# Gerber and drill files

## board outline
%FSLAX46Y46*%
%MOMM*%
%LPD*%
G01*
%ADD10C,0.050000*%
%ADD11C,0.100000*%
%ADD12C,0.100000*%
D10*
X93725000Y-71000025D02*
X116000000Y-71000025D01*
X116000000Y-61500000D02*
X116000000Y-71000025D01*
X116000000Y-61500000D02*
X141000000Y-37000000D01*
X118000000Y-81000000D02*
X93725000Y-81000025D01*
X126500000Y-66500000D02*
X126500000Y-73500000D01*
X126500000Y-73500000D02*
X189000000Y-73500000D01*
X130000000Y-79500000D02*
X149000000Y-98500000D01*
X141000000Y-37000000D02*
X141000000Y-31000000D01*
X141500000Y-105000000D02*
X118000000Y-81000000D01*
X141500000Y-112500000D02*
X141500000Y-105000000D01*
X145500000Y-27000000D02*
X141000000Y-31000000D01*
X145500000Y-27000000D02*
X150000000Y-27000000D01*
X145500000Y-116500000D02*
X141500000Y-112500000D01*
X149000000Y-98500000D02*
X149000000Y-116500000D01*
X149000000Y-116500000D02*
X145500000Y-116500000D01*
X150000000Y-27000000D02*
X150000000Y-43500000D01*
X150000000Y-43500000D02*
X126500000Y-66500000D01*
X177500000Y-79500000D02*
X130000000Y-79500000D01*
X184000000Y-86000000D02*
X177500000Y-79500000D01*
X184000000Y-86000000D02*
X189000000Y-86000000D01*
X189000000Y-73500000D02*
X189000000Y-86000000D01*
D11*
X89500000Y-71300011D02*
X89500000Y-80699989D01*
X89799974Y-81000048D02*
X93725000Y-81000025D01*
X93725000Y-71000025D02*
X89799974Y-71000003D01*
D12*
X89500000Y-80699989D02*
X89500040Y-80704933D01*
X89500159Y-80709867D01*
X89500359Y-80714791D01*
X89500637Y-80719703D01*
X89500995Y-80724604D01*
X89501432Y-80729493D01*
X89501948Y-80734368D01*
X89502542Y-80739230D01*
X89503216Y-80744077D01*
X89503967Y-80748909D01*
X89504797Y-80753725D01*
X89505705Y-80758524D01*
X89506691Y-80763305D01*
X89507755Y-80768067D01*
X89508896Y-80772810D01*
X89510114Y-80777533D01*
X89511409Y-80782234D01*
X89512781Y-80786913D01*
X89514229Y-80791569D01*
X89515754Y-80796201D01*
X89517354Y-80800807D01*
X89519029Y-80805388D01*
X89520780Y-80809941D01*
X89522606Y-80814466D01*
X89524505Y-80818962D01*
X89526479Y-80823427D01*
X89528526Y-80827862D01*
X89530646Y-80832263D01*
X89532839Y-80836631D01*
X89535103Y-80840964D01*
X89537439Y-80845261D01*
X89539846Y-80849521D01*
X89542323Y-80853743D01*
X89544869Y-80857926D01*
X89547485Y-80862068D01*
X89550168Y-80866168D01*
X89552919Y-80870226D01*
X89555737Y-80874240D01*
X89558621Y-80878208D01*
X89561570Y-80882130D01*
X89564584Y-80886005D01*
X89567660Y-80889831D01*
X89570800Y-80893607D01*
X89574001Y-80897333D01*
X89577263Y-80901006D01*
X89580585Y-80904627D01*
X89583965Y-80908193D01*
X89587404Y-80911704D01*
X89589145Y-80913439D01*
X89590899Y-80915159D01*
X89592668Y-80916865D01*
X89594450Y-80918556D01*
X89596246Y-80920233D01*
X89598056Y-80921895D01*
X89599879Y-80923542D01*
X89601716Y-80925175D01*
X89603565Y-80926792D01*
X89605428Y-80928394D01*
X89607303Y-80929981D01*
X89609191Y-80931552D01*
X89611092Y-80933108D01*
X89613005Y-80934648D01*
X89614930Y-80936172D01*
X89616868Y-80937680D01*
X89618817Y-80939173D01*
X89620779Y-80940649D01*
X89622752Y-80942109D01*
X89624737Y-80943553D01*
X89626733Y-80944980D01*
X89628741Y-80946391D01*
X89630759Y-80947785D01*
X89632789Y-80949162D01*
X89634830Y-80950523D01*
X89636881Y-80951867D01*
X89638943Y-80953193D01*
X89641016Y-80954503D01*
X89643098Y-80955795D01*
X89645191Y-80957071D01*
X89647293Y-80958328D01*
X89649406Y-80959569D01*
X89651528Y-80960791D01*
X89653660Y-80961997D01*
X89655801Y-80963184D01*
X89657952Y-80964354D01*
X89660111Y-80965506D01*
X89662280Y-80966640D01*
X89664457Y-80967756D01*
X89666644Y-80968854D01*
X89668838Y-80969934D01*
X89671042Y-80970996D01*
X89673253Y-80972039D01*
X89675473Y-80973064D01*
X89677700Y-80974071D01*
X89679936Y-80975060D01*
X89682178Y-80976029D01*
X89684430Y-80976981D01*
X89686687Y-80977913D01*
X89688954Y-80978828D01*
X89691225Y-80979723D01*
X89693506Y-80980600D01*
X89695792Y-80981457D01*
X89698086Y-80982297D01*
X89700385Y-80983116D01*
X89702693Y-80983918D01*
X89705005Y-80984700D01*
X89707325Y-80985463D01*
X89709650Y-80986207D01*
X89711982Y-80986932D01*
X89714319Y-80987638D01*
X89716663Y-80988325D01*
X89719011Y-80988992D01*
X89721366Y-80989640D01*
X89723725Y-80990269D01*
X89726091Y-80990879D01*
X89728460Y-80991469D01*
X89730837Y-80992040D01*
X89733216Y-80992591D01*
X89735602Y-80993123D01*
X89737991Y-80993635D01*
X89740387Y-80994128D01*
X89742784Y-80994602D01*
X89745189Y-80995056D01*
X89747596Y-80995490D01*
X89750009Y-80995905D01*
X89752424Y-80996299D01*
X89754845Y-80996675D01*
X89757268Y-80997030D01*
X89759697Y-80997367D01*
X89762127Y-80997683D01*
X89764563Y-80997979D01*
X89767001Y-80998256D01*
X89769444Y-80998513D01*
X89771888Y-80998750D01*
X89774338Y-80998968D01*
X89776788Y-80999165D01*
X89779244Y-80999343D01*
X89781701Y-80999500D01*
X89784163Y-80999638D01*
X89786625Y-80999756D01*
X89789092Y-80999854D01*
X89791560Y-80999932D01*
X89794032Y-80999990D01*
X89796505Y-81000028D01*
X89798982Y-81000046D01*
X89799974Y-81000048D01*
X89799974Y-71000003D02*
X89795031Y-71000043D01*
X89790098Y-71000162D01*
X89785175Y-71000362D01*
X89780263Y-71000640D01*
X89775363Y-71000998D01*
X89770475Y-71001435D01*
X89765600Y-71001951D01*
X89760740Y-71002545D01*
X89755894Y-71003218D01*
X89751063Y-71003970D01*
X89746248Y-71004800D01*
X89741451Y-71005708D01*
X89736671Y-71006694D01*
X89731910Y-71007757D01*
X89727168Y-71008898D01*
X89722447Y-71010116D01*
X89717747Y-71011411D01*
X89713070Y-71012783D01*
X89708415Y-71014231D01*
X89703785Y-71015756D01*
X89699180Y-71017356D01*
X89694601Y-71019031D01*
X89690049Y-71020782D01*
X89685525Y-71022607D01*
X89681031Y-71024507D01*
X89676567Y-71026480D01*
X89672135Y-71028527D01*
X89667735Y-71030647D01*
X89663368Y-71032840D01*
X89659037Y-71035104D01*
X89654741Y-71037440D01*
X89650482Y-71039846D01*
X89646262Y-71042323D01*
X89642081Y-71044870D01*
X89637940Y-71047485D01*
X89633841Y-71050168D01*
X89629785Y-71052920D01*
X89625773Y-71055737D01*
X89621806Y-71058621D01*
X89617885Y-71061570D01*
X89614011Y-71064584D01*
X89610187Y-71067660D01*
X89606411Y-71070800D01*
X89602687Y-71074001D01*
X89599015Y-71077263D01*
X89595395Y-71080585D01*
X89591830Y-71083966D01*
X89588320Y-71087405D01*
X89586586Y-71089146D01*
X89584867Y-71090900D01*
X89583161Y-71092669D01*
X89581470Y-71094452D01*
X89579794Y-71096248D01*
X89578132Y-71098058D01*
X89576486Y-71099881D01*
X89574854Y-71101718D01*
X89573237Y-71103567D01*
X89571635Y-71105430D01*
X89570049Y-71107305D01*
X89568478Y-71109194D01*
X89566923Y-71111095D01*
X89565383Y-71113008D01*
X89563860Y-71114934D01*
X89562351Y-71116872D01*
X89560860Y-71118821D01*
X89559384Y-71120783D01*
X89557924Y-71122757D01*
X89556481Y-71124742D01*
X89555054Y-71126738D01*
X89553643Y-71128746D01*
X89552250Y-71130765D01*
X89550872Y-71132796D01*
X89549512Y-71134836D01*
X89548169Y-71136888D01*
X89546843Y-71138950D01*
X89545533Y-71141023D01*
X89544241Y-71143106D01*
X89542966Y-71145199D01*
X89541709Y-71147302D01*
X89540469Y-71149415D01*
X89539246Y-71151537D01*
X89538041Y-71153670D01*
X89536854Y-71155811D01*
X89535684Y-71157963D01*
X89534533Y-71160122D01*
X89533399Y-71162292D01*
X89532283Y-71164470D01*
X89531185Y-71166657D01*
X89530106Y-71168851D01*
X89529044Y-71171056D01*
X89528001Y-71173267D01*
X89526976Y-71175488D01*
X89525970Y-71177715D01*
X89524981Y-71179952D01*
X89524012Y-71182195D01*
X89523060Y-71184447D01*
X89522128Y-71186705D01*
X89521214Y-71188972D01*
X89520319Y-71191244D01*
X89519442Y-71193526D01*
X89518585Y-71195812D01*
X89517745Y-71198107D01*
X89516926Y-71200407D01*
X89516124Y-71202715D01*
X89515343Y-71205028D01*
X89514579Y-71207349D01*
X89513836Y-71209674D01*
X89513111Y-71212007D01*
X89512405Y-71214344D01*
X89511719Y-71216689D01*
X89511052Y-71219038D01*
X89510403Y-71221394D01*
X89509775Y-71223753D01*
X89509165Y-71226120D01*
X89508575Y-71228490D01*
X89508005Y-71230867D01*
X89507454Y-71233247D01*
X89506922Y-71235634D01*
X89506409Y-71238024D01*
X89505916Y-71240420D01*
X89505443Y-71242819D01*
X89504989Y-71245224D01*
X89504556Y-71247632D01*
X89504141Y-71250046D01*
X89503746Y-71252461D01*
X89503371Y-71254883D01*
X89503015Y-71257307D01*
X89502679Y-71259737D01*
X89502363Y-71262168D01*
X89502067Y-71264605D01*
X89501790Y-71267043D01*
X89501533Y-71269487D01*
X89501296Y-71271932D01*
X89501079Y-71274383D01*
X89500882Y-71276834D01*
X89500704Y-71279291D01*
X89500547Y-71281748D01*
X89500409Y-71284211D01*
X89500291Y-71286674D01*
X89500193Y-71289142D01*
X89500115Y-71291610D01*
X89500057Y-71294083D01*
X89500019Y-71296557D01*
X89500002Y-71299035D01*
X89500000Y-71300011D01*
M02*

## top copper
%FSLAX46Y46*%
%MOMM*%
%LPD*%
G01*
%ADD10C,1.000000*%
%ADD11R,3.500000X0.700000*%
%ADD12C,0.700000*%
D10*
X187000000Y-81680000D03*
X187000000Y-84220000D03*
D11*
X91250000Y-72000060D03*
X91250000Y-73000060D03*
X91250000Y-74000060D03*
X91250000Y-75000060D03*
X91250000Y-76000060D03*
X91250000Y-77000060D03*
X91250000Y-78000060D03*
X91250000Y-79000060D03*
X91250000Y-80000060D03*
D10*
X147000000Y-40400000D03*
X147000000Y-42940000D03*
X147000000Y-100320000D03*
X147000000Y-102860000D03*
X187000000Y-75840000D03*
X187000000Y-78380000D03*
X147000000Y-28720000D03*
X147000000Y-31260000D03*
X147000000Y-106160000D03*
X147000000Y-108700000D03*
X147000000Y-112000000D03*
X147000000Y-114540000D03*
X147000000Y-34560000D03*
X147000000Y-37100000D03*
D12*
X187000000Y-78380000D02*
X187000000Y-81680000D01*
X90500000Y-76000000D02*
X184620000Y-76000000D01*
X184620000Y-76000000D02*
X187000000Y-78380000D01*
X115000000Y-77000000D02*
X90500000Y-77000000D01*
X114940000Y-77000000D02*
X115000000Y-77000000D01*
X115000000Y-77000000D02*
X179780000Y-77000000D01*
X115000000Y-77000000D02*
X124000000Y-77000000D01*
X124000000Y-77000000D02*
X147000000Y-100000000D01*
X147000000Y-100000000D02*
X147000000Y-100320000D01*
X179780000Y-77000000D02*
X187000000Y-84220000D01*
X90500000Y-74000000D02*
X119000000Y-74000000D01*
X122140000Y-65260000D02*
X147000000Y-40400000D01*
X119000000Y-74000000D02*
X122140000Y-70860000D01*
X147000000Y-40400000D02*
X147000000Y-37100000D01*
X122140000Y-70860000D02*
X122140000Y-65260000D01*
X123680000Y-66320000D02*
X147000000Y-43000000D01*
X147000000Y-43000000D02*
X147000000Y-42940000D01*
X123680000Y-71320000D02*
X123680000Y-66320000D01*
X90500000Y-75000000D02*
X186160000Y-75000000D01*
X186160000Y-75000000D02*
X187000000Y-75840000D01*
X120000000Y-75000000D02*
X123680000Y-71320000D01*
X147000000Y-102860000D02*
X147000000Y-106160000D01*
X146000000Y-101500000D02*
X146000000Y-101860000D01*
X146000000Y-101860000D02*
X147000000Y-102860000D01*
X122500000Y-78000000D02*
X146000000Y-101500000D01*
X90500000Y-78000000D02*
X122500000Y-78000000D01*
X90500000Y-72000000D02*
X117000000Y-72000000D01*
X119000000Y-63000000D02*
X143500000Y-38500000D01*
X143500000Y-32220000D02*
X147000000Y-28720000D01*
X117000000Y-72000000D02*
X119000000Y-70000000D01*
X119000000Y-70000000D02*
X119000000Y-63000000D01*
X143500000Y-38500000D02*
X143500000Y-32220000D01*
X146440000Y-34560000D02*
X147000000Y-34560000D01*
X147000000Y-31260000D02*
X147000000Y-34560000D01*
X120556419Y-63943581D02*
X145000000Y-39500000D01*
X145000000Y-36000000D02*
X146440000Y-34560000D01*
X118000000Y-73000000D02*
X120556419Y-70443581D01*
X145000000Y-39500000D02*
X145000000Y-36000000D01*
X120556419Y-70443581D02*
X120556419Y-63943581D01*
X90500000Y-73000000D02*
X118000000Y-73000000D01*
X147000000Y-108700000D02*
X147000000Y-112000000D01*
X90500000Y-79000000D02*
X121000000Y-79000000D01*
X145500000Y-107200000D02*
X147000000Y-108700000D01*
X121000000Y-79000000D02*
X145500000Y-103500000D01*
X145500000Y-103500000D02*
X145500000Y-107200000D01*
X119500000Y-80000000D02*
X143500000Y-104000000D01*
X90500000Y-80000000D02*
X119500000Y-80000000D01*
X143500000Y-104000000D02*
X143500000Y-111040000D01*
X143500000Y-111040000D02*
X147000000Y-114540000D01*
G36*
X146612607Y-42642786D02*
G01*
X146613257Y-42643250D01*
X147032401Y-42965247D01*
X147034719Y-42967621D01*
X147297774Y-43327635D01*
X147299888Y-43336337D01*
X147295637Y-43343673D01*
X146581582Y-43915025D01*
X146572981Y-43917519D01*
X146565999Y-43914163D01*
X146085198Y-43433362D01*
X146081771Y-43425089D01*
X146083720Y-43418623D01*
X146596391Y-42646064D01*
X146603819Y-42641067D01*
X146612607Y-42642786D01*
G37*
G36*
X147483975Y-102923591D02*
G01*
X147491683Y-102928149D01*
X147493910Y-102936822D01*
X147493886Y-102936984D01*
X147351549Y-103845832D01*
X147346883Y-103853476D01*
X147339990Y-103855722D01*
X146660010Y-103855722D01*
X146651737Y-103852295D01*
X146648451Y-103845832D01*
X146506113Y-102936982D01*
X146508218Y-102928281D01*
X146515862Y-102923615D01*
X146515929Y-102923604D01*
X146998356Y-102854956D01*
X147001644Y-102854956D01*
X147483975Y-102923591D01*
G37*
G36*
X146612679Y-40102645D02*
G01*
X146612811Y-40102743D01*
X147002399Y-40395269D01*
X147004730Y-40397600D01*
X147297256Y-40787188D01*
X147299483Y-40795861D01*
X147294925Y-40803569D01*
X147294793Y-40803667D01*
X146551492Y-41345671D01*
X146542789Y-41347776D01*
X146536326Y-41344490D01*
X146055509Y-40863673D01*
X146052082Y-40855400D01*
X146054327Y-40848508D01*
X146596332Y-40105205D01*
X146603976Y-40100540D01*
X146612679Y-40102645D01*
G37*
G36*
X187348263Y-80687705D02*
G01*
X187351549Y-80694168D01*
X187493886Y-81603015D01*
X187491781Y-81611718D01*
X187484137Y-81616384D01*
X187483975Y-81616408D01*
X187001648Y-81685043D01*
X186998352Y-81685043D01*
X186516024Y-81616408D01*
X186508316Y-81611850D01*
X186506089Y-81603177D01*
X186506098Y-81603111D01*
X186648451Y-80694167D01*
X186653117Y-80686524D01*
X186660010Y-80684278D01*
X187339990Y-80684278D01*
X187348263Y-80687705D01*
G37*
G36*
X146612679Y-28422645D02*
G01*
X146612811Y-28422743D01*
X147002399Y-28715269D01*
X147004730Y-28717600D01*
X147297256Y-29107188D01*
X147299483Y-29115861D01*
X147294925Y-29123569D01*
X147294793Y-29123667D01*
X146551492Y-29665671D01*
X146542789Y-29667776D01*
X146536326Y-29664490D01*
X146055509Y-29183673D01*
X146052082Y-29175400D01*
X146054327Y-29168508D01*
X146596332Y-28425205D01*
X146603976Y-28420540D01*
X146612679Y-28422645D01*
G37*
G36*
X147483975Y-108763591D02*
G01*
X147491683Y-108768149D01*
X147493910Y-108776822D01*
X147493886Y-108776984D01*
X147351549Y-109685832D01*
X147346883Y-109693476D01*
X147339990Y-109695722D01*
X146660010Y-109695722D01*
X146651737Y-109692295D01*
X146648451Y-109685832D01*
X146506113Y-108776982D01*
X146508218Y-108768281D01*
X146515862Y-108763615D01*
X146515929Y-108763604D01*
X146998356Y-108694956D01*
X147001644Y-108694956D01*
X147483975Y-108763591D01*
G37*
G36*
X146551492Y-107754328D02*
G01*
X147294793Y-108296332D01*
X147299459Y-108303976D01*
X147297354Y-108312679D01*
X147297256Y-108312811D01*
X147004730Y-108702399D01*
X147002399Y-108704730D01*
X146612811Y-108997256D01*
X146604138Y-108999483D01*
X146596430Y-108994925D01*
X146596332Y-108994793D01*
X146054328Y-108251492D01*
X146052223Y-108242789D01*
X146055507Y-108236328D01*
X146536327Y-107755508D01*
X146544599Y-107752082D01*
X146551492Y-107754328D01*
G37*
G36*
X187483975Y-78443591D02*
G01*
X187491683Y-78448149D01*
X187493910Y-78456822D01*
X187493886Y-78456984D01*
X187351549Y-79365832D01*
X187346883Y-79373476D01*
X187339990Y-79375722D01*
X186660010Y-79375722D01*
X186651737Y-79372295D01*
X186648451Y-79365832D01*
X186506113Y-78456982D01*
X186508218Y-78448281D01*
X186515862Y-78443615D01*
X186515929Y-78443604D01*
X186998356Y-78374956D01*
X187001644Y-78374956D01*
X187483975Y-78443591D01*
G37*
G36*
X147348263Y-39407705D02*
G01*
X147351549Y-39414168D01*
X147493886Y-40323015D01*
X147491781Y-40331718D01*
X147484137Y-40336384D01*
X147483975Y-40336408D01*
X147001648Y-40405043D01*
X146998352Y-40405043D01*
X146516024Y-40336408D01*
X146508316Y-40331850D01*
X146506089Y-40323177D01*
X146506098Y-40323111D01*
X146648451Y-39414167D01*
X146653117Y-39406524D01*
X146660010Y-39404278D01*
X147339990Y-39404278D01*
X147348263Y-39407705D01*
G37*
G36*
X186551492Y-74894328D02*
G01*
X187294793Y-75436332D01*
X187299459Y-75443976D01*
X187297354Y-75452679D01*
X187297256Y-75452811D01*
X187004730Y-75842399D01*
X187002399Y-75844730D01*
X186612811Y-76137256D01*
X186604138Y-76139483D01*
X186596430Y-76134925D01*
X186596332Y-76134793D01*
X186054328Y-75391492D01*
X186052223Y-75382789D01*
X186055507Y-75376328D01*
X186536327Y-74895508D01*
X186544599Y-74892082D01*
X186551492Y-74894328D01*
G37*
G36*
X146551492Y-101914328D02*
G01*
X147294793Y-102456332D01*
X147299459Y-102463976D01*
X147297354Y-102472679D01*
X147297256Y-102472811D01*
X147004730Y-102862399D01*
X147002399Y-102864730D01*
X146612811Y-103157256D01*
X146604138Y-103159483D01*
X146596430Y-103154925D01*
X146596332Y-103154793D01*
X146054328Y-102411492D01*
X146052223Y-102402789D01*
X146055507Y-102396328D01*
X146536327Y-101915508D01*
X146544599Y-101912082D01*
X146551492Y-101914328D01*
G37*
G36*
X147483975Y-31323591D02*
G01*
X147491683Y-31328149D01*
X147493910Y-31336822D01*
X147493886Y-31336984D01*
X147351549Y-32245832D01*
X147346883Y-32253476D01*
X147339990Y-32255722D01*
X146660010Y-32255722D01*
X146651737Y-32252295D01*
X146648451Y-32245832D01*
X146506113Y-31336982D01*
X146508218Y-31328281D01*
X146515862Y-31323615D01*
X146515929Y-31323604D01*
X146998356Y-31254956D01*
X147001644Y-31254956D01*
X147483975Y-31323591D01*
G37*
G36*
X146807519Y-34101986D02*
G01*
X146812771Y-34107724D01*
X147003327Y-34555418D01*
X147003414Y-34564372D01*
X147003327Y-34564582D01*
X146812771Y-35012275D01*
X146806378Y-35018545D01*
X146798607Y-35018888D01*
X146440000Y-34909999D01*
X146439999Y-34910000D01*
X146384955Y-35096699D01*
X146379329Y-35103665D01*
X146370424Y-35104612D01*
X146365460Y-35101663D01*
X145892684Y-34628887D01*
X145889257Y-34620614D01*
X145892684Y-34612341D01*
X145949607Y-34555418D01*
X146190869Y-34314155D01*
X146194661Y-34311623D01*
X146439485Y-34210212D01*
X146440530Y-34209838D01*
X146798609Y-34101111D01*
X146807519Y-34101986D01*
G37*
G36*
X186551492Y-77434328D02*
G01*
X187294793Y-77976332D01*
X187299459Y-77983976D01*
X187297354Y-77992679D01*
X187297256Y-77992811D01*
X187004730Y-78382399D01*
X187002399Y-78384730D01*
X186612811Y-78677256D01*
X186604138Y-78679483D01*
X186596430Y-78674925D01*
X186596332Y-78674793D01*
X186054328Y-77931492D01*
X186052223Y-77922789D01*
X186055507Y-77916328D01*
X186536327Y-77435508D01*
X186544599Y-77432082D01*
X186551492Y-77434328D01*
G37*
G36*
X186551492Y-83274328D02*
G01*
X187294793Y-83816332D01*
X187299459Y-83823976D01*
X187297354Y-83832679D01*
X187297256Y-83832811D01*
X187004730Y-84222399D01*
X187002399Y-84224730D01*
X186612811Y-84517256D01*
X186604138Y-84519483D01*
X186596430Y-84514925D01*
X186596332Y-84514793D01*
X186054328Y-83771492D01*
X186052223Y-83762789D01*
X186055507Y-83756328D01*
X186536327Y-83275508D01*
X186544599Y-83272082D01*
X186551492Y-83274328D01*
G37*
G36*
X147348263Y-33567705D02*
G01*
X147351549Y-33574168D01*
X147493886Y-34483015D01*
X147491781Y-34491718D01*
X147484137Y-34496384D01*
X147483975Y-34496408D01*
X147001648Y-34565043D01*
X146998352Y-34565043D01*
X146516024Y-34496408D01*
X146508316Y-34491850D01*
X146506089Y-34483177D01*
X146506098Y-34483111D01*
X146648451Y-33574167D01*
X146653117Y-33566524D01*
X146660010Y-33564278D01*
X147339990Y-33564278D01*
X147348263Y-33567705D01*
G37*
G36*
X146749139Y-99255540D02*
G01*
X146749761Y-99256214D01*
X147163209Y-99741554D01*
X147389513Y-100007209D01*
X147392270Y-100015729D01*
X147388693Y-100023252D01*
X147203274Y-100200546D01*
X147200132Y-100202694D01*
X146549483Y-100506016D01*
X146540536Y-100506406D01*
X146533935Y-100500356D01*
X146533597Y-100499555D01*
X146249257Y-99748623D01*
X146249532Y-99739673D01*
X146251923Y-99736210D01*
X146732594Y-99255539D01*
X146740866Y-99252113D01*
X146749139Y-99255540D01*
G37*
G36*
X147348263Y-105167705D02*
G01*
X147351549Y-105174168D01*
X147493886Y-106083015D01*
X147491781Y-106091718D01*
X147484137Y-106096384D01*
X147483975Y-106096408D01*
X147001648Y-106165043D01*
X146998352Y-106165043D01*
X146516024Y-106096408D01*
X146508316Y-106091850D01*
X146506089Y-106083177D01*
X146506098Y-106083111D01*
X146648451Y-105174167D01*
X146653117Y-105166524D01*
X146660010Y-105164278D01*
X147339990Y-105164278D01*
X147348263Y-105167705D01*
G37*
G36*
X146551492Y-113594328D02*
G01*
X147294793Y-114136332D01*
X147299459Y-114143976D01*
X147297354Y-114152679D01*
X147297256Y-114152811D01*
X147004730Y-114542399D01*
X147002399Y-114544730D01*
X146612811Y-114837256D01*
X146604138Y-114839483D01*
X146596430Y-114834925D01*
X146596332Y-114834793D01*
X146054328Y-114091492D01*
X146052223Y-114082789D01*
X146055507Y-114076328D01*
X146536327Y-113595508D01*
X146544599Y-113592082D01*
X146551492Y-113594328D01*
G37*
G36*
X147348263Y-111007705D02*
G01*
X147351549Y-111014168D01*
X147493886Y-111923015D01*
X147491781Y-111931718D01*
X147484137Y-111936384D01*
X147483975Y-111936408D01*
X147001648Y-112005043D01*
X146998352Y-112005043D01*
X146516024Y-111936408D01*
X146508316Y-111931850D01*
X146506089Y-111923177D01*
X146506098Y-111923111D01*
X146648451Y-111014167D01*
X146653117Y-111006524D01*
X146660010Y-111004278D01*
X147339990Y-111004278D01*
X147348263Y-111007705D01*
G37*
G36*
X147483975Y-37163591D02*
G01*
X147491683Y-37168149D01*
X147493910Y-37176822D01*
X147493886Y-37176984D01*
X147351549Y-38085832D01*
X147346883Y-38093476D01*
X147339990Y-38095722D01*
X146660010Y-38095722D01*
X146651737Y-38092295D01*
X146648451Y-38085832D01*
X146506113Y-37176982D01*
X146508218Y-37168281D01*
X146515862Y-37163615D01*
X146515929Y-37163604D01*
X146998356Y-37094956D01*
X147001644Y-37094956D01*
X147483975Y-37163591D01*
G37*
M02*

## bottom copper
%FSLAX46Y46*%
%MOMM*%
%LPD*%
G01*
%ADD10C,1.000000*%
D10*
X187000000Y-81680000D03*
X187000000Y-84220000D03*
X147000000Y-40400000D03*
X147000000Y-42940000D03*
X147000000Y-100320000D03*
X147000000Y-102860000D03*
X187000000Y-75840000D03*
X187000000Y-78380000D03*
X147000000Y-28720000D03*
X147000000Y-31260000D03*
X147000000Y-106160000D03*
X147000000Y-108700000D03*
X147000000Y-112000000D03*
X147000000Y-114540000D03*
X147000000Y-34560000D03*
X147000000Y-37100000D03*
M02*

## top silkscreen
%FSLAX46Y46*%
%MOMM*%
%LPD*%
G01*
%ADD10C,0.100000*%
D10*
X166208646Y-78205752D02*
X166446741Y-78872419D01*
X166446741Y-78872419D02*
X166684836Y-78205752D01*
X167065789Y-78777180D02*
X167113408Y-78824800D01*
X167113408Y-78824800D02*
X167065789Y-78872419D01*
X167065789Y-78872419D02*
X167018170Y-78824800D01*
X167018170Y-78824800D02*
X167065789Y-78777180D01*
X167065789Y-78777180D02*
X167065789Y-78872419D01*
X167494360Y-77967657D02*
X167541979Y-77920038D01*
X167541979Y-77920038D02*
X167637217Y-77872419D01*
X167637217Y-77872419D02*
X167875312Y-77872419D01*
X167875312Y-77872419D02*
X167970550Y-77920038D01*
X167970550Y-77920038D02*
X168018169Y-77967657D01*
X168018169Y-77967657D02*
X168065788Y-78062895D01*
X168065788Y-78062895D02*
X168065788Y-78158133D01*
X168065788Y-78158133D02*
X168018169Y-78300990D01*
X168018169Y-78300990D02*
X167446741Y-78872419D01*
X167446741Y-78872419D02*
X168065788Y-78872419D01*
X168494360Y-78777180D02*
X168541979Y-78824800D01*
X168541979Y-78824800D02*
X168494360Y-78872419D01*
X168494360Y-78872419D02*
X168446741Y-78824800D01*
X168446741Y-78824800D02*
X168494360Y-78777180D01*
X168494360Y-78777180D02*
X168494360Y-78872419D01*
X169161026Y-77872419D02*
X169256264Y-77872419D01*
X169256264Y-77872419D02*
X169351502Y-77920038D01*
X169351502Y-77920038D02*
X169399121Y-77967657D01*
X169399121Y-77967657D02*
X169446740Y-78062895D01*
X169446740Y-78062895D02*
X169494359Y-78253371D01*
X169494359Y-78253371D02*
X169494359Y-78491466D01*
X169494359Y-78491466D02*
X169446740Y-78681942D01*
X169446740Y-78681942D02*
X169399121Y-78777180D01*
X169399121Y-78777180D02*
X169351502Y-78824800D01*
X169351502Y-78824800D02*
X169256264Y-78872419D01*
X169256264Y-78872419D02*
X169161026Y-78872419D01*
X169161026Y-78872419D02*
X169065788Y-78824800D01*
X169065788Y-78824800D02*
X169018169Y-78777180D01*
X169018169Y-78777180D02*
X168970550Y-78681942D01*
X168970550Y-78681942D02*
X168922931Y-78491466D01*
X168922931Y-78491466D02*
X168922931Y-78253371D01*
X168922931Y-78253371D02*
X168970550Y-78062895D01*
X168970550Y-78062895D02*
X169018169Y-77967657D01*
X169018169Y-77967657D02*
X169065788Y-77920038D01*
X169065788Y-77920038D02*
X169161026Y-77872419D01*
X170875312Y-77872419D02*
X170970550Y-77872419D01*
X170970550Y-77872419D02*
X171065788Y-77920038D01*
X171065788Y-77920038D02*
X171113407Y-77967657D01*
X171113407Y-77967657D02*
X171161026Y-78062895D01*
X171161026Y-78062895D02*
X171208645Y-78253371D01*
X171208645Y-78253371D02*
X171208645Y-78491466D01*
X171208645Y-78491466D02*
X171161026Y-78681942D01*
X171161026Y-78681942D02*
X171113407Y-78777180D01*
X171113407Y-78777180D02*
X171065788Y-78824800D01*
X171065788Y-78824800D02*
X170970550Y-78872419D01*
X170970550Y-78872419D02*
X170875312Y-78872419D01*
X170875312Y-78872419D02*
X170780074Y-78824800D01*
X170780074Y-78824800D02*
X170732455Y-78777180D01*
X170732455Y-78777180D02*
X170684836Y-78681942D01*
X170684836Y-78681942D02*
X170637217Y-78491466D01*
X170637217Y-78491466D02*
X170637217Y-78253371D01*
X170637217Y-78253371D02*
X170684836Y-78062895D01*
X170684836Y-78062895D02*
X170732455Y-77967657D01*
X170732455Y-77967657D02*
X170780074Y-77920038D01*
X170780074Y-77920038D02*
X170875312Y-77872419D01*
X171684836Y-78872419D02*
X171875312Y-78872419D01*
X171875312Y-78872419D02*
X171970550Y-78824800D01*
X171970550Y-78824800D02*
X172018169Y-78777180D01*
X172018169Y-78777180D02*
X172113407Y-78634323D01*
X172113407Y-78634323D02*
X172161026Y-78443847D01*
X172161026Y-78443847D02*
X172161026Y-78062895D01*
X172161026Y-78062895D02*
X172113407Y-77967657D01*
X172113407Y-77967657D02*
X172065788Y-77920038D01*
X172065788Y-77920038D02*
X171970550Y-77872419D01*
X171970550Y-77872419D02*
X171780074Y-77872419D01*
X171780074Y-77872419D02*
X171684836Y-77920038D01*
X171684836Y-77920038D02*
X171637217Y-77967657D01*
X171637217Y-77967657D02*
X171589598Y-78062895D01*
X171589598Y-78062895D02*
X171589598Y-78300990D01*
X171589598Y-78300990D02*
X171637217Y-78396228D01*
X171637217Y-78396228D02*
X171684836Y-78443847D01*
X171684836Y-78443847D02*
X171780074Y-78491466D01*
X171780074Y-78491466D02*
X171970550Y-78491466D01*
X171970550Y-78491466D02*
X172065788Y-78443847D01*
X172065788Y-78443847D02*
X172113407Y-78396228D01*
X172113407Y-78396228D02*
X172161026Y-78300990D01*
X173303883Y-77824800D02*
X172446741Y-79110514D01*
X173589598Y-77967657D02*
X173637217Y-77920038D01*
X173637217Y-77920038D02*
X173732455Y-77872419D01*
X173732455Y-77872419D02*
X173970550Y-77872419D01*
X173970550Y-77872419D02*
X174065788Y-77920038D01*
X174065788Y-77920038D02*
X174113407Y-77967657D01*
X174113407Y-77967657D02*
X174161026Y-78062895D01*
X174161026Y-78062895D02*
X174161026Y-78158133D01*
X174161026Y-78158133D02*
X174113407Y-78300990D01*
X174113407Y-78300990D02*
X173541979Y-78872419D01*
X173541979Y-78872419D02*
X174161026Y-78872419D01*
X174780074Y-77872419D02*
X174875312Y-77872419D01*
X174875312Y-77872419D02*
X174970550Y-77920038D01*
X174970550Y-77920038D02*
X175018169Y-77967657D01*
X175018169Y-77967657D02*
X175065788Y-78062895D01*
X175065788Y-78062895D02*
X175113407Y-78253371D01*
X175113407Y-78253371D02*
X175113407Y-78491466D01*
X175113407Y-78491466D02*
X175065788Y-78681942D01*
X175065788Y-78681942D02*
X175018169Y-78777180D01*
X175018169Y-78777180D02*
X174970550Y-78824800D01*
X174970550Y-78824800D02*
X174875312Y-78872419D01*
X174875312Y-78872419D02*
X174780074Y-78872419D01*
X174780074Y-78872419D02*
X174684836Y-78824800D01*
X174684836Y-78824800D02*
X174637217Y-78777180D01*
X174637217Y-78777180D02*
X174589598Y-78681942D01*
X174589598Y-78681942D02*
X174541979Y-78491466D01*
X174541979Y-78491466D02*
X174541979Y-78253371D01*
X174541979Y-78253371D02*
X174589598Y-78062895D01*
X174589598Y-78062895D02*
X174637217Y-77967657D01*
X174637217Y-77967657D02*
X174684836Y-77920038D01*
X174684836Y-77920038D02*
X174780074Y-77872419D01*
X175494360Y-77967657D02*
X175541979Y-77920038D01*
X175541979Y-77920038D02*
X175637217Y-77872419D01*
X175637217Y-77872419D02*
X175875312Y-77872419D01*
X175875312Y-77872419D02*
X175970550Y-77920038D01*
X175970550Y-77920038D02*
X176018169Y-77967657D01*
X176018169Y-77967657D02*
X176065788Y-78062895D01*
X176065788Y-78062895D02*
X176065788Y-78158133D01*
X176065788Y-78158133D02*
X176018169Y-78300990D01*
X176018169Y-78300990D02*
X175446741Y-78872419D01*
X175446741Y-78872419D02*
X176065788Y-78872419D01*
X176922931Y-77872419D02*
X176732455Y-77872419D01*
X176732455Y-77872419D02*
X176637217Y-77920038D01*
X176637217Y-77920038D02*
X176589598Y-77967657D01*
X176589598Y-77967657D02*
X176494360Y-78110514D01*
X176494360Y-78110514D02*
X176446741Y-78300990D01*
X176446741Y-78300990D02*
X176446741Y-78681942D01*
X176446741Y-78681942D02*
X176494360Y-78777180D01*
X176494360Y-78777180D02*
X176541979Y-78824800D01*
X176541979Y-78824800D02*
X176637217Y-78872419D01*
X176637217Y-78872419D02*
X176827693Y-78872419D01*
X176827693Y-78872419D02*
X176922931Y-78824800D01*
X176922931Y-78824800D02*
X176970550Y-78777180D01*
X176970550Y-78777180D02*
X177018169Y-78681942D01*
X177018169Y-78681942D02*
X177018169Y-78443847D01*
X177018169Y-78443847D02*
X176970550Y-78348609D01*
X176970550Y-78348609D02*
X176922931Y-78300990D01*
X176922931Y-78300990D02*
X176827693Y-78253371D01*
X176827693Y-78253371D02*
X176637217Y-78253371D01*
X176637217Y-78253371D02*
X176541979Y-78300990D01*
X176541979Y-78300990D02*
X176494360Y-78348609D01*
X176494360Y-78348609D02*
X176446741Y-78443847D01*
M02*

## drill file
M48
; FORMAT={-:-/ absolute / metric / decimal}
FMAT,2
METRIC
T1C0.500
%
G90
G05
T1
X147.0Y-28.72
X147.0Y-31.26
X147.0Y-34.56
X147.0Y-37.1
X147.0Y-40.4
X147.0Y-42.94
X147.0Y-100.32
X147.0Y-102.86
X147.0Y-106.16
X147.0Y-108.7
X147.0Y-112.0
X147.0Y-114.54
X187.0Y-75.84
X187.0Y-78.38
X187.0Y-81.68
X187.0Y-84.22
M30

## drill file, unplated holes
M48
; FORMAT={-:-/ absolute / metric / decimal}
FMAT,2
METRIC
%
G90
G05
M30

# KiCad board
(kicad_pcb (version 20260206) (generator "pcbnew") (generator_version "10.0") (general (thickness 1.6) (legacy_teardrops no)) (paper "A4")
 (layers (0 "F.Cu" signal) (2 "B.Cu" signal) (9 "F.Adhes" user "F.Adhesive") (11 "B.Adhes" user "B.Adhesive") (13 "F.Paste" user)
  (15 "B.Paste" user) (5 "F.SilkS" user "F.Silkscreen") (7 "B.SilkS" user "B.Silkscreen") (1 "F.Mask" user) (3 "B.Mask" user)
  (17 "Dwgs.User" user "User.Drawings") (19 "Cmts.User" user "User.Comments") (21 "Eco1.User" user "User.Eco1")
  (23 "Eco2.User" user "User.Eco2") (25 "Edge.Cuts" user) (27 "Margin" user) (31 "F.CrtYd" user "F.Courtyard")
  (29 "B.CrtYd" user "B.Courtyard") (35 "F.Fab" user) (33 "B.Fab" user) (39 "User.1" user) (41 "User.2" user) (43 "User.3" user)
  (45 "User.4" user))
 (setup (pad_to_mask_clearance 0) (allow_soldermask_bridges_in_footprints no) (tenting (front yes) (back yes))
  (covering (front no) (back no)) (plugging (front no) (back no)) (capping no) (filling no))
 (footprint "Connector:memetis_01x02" (layer "F.Cu") (at 189.5 88.95)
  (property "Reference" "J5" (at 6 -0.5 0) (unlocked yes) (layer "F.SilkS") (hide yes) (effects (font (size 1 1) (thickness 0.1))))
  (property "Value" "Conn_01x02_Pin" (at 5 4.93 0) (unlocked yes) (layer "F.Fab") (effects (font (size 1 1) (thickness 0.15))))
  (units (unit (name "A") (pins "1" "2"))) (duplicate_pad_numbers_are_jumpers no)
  (pad "1" thru_hole circle (at -2.5 -7.27) (size 1 1) (drill 0.5) (layers "*.Cu" "*.Mask") (remove_unused_layers no) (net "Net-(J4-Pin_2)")
   (teardrops (best_length_ratio 0.5) (max_length 1) (best_width_ratio 1) (max_width 2) (curved_edges no) (filter_ratio 0.9) (enabled yes)
    (allow_two_segments yes) (prefer_zone_connections yes)))
  (pad "2" thru_hole circle (at -2.5 -4.73) (size 1 1) (drill 0.5) (layers "*.Cu" "*.Mask") (remove_unused_layers no) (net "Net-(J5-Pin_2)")
   (teardrops (best_length_ratio 0.5) (max_length 1) (best_width_ratio 1) (max_width 2) (curved_edges no) (filter_ratio 0.9) (enabled yes)
    (allow_two_segments yes) (prefer_zone_connections yes))))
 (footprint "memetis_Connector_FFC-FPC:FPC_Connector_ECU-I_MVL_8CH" (layer "F.Cu") (at 91.6125 76.000025)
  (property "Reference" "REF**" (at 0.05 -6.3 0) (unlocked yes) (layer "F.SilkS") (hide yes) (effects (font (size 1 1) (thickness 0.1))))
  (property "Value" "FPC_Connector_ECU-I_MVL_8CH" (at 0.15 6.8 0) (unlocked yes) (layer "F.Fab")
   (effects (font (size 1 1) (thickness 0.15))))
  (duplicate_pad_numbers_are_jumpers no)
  (fp_line (start -2.1125 -4.700014) (end -2.1125 4.699964) (stroke (width 0.1) (type default)) (layer "Edge.Cuts"))
  (fp_line (start -1.812526 5.000023) (end 2.1125 5) (stroke (width 0.1) (type default)) (layer "Edge.Cuts"))
  (fp_line (start 2.1125 -5) (end -1.812526 -5.000022) (stroke (width 0.1) (type default)) (layer "Edge.Cuts"))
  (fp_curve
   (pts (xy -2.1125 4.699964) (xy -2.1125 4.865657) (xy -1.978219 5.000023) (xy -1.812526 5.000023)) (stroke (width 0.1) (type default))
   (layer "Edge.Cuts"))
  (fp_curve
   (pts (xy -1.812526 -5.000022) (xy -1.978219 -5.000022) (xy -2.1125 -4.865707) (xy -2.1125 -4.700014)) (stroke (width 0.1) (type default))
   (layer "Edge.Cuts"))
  (pad "1" smd rect (at -0.3625 -3.999965 270) (size 0.7 3.5) (layers "F.Cu" "F.Mask" "F.Paste") (clearance 0.25)
   (teardrops (best_length_ratio 0.5) (max_length 1) (best_width_ratio 1) (max_width 2) (curved_edges no) (filter_ratio 0.9) (enabled yes)
    (allow_two_segments yes) (prefer_zone_connections yes)))
  (pad "2" smd rect (at -0.3625 -2.999965 270) (size 0.7 3.5) (layers "F.Cu" "F.Mask" "F.Paste") (clearance 0.25)
   (teardrops (best_length_ratio 0.5) (max_length 1) (best_width_ratio 1) (max_width 2) (curved_edges no) (filter_ratio 0.9) (enabled yes)
    (allow_two_segments yes) (prefer_zone_connections yes)))
  (pad "3" smd rect (at -0.3625 -1.999965 270) (size 0.7 3.5) (layers "F.Cu" "F.Mask" "F.Paste") (clearance 0.25)
   (teardrops (best_length_ratio 0.5) (max_length 1) (best_width_ratio 1) (max_width 2) (curved_edges no) (filter_ratio 0.9) (enabled yes)
    (allow_two_segments yes) (prefer_zone_connections yes)))
  (pad "4" smd rect (at -0.3625 -0.999965 270) (size 0.7 3.5) (layers "F.Cu" "F.Mask" "F.Paste") (clearance 0.25)
   (teardrops (best_length_ratio 0.5) (max_length 1) (best_width_ratio 1) (max_width 2) (curved_edges no) (filter_ratio 0.9) (enabled yes)
    (allow_two_segments yes) (prefer_zone_connections yes)))
  (pad "5" smd rect (at -0.3625 0.000035 270) (size 0.7 3.5) (layers "F.Cu" "F.Mask" "F.Paste") (clearance 0.25)
   (teardrops (best_length_ratio 0.5) (max_length 1) (best_width_ratio 1) (max_width 2) (curved_edges no) (filter_ratio 0.9) (enabled yes)
    (allow_two_segments yes) (prefer_zone_connections yes)))
  (pad "6" smd rect (at -0.3625 1.000035 270) (size 0.7 3.5) (layers "F.Cu" "F.Mask" "F.Paste") (clearance 0.25)
   (teardrops (best_length_ratio 0.5) (max_length 1) (best_width_ratio 1) (max_width 2) (curved_edges no) (filter_ratio 0.9) (enabled yes)
    (allow_two_segments yes) (prefer_zone_connections yes)))
  (pad "7" smd rect (at -0.3625 2.000035 270) (size 0.7 3.5) (layers "F.Cu" "F.Mask" "F.Paste") (clearance 0.25)
   (teardrops (best_length_ratio 0.5) (max_length 1) (best_width_ratio 1) (max_width 2) (curved_edges no) (filter_ratio 0.9) (enabled yes)
    (allow_two_segments yes) (prefer_zone_connections yes)))
  (pad "8" smd rect (at -0.3625 3.000035 90) (size 0.7 3.5) (layers "F.Cu" "F.Mask" "F.Paste") (clearance 0.25)
   (teardrops (best_length_ratio 0.5) (max_length 1) (best_width_ratio 1) (max_width 2) (curved_edges no) (filter_ratio 0.9) (enabled yes)
    (allow_two_segments yes) (prefer_zone_connections yes)))
  (pad "9" smd rect (at -0.3625 4.000035 270) (size 0.7 3.5) (layers "F.Cu" "F.Mask" "F.Paste") (clearance 0.25)
   (teardrops (best_length_ratio 0.5) (max_length 1) (best_width_ratio 1) (max_width 2) (curved_edges no) (filter_ratio 0.9) (enabled yes)
    (allow_two_segments yes) (prefer_zone_connections yes))))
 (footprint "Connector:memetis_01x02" (layer "F.Cu") (at 149.5 47.67)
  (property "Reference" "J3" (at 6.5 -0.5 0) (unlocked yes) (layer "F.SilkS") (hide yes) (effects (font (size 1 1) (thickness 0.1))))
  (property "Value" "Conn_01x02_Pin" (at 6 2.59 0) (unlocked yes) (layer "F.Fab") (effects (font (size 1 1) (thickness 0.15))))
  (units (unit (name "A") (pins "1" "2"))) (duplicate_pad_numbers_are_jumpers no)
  (pad "1" thru_hole circle (at -2.5 -7.27) (size 1 1) (drill 0.5) (layers "*.Cu" "*.Mask") (remove_unused_layers no) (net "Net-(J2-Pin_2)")
   (teardrops (best_length_ratio 0.5) (max_length 1) (best_width_ratio 1) (max_width 2) (curved_edges no) (filter_ratio 0.9) (enabled yes)
    (allow_two_segments yes) (prefer_zone_connections yes)))
  (pad "2" thru_hole circle (at -2.5 -4.73) (size 1 1) (drill 0.5) (layers "*.Cu" "*.Mask") (remove_unused_layers no) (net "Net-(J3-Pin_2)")
   (teardrops (best_length_ratio 0.5) (max_length 1) (best_width_ratio 1) (max_width 2) (curved_edges no) (filter_ratio 0.9) (enabled yes)
    (allow_two_segments yes) (prefer_zone_connections yes))))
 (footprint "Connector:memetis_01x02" (layer "F.Cu") (at 149.5 107.59)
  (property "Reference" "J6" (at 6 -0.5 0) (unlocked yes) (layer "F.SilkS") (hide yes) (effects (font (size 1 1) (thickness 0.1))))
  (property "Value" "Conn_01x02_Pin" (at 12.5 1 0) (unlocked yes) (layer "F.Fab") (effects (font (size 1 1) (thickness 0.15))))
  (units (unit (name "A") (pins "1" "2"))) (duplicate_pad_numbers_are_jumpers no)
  (pad "1" thru_hole circle (at -2.5 -7.27) (size 1 1) (drill 0.5) (layers "*.Cu" "*.Mask") (remove_unused_layers no) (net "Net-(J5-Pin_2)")
   (teardrops (best_length_ratio 0.5) (max_length 1) (best_width_ratio 1) (max_width 2) (curved_edges no) (filter_ratio 0.9) (enabled yes)
    (allow_two_segments yes) (prefer_zone_connections yes)))
  (pad "2" thru_hole circle (at -2.5 -4.73) (size 1 1) (drill 0.5) (layers "*.Cu" "*.Mask") (remove_unused_layers no) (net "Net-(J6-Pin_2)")
   (teardrops (best_length_ratio 0.5) (max_length 1) (best_width_ratio 1) (max_width 2) (curved_edges no) (filter_ratio 0.9) (enabled yes)
    (allow_two_segments yes) (prefer_zone_connections yes))))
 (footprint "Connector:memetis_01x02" (layer "F.Cu") (at 189.5 83.11)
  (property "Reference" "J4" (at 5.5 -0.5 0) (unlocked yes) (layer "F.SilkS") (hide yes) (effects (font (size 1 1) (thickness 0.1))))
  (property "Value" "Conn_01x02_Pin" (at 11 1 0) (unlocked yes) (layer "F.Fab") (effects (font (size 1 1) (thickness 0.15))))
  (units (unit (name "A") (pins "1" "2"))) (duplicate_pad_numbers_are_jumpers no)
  (pad "1" thru_hole circle (at -2.5 -7.27) (size 1 1) (drill 0.5) (layers "*.Cu" "*.Mask") (remove_unused_layers no) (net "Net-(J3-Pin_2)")
   (teardrops (best_length_ratio 0.5) (max_length 1) (best_width_ratio 1) (max_width 2) (curved_edges no) (filter_ratio 0.9) (enabled yes)
    (allow_two_segments yes) (prefer_zone_connections yes)))
  (pad "2" thru_hole circle (at -2.5 -4.73) (size 1 1) (drill 0.5) (layers "*.Cu" "*.Mask") (remove_unused_layers no) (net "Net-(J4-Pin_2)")
   (teardrops (best_length_ratio 0.5) (max_length 1) (best_width_ratio 1) (max_width 2) (curved_edges no) (filter_ratio 0.9) (enabled yes)
    (allow_two_segments yes) (prefer_zone_connections yes))))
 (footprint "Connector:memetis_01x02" (layer "F.Cu") (at 149.5 35.99)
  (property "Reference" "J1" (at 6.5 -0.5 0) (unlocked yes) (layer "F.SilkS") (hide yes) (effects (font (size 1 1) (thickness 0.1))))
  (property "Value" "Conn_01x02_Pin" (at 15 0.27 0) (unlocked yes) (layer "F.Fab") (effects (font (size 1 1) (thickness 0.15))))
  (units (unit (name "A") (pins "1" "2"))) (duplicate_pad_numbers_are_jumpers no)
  (pad "1" thru_hole circle (at -2.5 -7.27) (size 1 1) (drill 0.5) (layers "*.Cu" "*.Mask") (remove_unused_layers no) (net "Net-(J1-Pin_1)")
   (teardrops (best_length_ratio 0.5) (max_length 1) (best_width_ratio 1) (max_width 2) (curved_edges no) (filter_ratio 0.9) (enabled yes)
    (allow_two_segments yes) (prefer_zone_connections yes)))
  (pad "2" thru_hole circle (at -2.5 -4.73) (size 1 1) (drill 0.5) (layers "*.Cu" "*.Mask") (remove_unused_layers no) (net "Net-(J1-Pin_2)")
   (teardrops (best_length_ratio 0.5) (max_length 1) (best_width_ratio 1) (max_width 2) (curved_edges no) (filter_ratio 0.9) (enabled yes)
    (allow_two_segments yes) (prefer_zone_connections yes))))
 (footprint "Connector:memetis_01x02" (layer "F.Cu") (at 149.5 113.43)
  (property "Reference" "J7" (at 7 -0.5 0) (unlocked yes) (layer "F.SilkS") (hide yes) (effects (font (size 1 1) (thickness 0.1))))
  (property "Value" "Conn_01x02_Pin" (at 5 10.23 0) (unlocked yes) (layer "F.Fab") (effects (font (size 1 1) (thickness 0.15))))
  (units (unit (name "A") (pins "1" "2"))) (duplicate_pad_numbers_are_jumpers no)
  (pad "1" thru_hole circle (at -2.5 -7.27) (size 1 1) (drill 0.5) (layers "*.Cu" "*.Mask") (remove_unused_layers no) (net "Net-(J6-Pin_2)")
   (teardrops (best_length_ratio 0.5) (max_length 1) (best_width_ratio 1) (max_width 2) (curved_edges no) (filter_ratio 0.9) (enabled yes)
    (allow_two_segments yes) (prefer_zone_connections yes)))
  (pad "2" thru_hole circle (at -2.5 -4.73) (size 1 1) (drill 0.5) (layers "*.Cu" "*.Mask") (remove_unused_layers no) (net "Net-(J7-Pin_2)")
   (teardrops (best_length_ratio 0.5) (max_length 1) (best_width_ratio 1) (max_width 2) (curved_edges no) (filter_ratio 0.9) (enabled yes)
    (allow_two_segments yes) (prefer_zone_connections yes))))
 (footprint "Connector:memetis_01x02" (layer "F.Cu") (at 149.5 119.27)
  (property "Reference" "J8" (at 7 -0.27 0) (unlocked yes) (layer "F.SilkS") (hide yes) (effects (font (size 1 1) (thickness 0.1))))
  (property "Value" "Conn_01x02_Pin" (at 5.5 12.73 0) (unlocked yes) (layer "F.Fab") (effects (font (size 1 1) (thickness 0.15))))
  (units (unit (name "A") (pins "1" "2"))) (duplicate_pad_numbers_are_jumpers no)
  (pad "1" thru_hole circle (at -2.5 -7.27) (size 1 1) (drill 0.5) (layers "*.Cu" "*.Mask") (remove_unused_layers no) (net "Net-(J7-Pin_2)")
   (teardrops (best_length_ratio 0.5) (max_length 1) (best_width_ratio 1) (max_width 2) (curved_edges no) (filter_ratio 0.9) (enabled yes)
    (allow_two_segments yes) (prefer_zone_connections yes)))
  (pad "2" thru_hole circle (at -2.5 -4.73) (size 1 1) (drill 0.5) (layers "*.Cu" "*.Mask") (remove_unused_layers no) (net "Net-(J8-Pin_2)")
   (teardrops (best_length_ratio 0.5) (max_length 1) (best_width_ratio 1) (max_width 2) (curved_edges no) (filter_ratio 0.9) (enabled yes)
    (allow_two_segments yes) (prefer_zone_connections yes))))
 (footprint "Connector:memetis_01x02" (layer "F.Cu") (at 149.5 41.83)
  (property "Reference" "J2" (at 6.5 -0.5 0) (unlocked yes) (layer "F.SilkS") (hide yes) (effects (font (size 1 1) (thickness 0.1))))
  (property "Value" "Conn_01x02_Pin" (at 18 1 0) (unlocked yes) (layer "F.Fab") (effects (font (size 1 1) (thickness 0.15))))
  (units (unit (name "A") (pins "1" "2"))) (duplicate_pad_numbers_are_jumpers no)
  (pad "1" thru_hole circle (at -2.5 -7.27) (size 1 1) (drill 0.5) (layers "*.Cu" "*.Mask") (remove_unused_layers no) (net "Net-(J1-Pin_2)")
   (teardrops (best_length_ratio 0.5) (max_length 1) (best_width_ratio 1) (max_width 2) (curved_edges no) (filter_ratio 0.9) (enabled yes)
    (allow_two_segments yes) (prefer_zone_connections yes)))
  (pad "2" thru_hole circle (at -2.5 -4.73) (size 1 1) (drill 0.5) (layers "*.Cu" "*.Mask") (remove_unused_layers no) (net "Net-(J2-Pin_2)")
   (teardrops (best_length_ratio 0.5) (max_length 1) (best_width_ratio 1) (max_width 2) (curved_edges no) (filter_ratio 0.9) (enabled yes)
    (allow_two_segments yes) (prefer_zone_connections yes))))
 (gr_line (start 93.725 71.000025) (end 116 71.000025) (stroke (width 0.05) (type default)) (layer "Edge.Cuts"))
 (gr_line (start 116 61.5) (end 116 71.000025) (stroke (width 0.05) (type default)) (layer "Edge.Cuts"))
 (gr_line (start 116 61.5) (end 141 37) (stroke (width 0.05) (type default)) (layer "Edge.Cuts"))
 (gr_line (start 118 81) (end 93.725 81.000025) (stroke (width 0.05) (type default)) (layer "Edge.Cuts"))
 (gr_line (start 126.5 66.5) (end 126.5 73.5) (stroke (width 0.05) (type default)) (layer "Edge.Cuts"))
 (gr_line (start 126.5 73.5) (end 189 73.5) (stroke (width 0.05) (type default)) (layer "Edge.Cuts"))
 (gr_line (start 130 79.5) (end 149 98.5) (stroke (width 0.05) (type default)) (layer "Edge.Cuts"))
 (gr_line (start 141 37) (end 141 31) (stroke (width 0.05) (type default)) (layer "Edge.Cuts"))
 (gr_line (start 141.5 105) (end 118 81) (stroke (width 0.05) (type default)) (layer "Edge.Cuts"))
 (gr_line (start 141.5 112.5) (end 141.5 105) (stroke (width 0.05) (type default)) (layer "Edge.Cuts"))
 (gr_line (start 145.5 27) (end 141 31) (stroke (width 0.05) (type default)) (layer "Edge.Cuts"))
 (gr_line (start 145.5 27) (end 150 27) (stroke (width 0.05) (type default)) (layer "Edge.Cuts"))
 (gr_line (start 145.5 116.5) (end 141.5 112.5) (stroke (width 0.05) (type default)) (layer "Edge.Cuts"))
 (gr_line (start 149 98.5) (end 149 116.5) (stroke (width 0.05) (type default)) (layer "Edge.Cuts"))
 (gr_line (start 149 116.5) (end 145.5 116.5) (stroke (width 0.05) (type default)) (layer "Edge.Cuts"))
 (gr_line (start 150 27) (end 150 43.5) (stroke (width 0.05) (type default)) (layer "Edge.Cuts"))
 (gr_line (start 150 43.5) (end 126.5 66.5) (stroke (width 0.05) (type default)) (layer "Edge.Cuts"))
 (gr_line (start 177.5 79.5) (end 130 79.5) (stroke (width 0.05) (type default)) (layer "Edge.Cuts"))
 (gr_line (start 184 86) (end 177.5 79.5) (stroke (width 0.05) (type default)) (layer "Edge.Cuts"))
 (gr_line (start 184 86) (end 189 86) (stroke (width 0.05) (type default)) (layer "Edge.Cuts"))
 (gr_line (start 189 73.5) (end 189 86) (stroke (width 0.05) (type default)) (layer "Edge.Cuts"))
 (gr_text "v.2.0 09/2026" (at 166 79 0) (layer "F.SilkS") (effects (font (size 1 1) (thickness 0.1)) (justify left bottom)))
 (segment (start 187 78.38) (end 187 81.68) (width 0.7) (layer "F.Cu") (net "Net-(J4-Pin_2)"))
 (segment (start 90.5 76) (end 184.62 76) (width 0.7) (layer "F.Cu") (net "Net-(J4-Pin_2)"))
 (segment (start 184.62 76) (end 187 78.38) (width 0.7) (layer "F.Cu") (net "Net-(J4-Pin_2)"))
 (segment (start 115 77) (end 90.5 77) (width 0.7) (layer "F.Cu") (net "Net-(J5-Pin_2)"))
 (segment (start 114.94 77) (end 115 77) (width 0.7) (layer "F.Cu") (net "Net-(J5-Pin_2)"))
 (segment (start 115 77) (end 179.78 77) (width 0.7) (layer "F.Cu") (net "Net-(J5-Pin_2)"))
 (segment (start 115 77) (end 124 77) (width 0.7) (layer "F.Cu") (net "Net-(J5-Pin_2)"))
 (segment (start 124 77) (end 147 100) (width 0.7) (layer "F.Cu") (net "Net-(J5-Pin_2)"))
 (segment (start 147 100) (end 147 100.32) (width 0.7) (layer "F.Cu") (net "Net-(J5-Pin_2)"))
 (segment (start 179.78 77) (end 187 84.22) (width 0.7) (layer "F.Cu") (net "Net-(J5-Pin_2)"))
 (segment (start 90.5 74) (end 119 74) (width 0.7) (layer "F.Cu") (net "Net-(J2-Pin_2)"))
 (segment (start 122.14 65.26) (end 147 40.4) (width 0.7) (layer "F.Cu") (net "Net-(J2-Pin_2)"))
 (segment (start 119 74) (end 122.14 70.86) (width 0.7) (layer "F.Cu") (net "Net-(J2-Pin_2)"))
 (segment (start 147 40.4) (end 147 37.1) (width 0.7) (layer "F.Cu") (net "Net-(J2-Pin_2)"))
 (segment (start 122.14 70.86) (end 122.14 65.26) (width 0.7) (layer "F.Cu") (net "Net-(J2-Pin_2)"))
 (segment (start 123.68 66.32) (end 147 43) (width 0.7) (layer "F.Cu") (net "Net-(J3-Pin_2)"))
 (segment (start 147 43) (end 147 42.94) (width 0.7) (layer "F.Cu") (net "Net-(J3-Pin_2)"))
 (segment (start 123.68 71.32) (end 123.68 66.32) (width 0.7) (layer "F.Cu") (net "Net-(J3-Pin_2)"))
 (segment (start 90.5 75) (end 186.16 75) (width 0.7) (layer "F.Cu") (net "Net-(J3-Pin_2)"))
 (segment (start 186.16 75) (end 187 75.84) (width 0.7) (layer "F.Cu") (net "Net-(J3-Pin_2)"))
 (segment (start 120 75) (end 123.68 71.32) (width 0.7) (layer "F.Cu") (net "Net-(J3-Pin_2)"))
 (segment (start 147 102.86) (end 147 106.16) (width 0.7) (layer "F.Cu") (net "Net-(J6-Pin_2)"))
 (segment (start 146 101.5) (end 146 101.86) (width 0.7) (layer "F.Cu") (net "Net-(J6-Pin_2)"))
 (segment (start 146 101.86) (end 147 102.86) (width 0.7) (layer "F.Cu") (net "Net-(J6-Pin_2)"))
 (segment (start 122.5 78) (end 146 101.5) (width 0.7) (layer "F.Cu") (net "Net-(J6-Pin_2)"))
 (segment (start 90.5 78) (end 122.5 78) (width 0.7) (layer "F.Cu") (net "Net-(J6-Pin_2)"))
 (segment (start 90.5 72) (end 117 72) (width 0.7) (layer "F.Cu") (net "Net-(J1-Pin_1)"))
 (segment (start 119 63) (end 143.5 38.5) (width 0.7) (layer "F.Cu") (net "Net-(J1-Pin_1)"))
 (segment (start 143.5 32.22) (end 147 28.72) (width 0.7) (layer "F.Cu") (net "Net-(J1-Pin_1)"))
 (segment (start 117 72) (end 119 70) (width 0.7) (layer "F.Cu") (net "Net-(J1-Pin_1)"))
 (segment (start 119 70) (end 119 63) (width 0.7) (layer "F.Cu") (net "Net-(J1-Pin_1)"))
 (segment (start 143.5 38.5) (end 143.5 32.22) (width 0.7) (layer "F.Cu") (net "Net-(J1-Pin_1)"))
 (segment (start 146.44 34.56) (end 147 34.56) (width 0.7) (layer "F.Cu") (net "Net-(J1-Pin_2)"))
 (segment (start 147 31.26) (end 147 34.56) (width 0.7) (layer "F.Cu") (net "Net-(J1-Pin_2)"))
 (segment (start 120.556419 63.943581) (end 145 39.5) (width 0.7) (layer "F.Cu") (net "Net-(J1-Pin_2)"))
 (segment (start 145 36) (end 146.44 34.56) (width 0.7) (layer "F.Cu") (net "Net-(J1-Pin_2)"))
 (segment (start 118 73) (end 120.556419 70.443581) (width 0.7) (layer "F.Cu") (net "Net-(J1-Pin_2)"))
 (segment (start 145 39.5) (end 145 36) (width 0.7) (layer "F.Cu") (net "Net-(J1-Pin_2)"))
 (segment (start 120.556419 70.443581) (end 120.556419 63.943581) (width 0.7) (layer "F.Cu") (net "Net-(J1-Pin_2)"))
 (segment (start 90.5 73) (end 118 73) (width 0.7) (layer "F.Cu") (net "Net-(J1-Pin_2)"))
 (segment (start 147 108.7) (end 147 112) (width 0.7) (layer "F.Cu") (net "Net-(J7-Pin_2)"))
 (segment (start 90.5 79) (end 121 79) (width 0.7) (layer "F.Cu") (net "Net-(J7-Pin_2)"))
 (segment (start 145.5 107.2) (end 147 108.7) (width 0.7) (layer "F.Cu") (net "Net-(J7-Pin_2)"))
 (segment (start 121 79) (end 145.5 103.5) (width 0.7) (layer "F.Cu") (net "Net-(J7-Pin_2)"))
 (segment (start 145.5 103.5) (end 145.5 107.2) (width 0.7) (layer "F.Cu") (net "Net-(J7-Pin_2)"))
 (segment (start 119.5 80) (end 143.5 104) (width 0.7) (layer "F.Cu") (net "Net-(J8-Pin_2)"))
 (segment (start 90.5 80) (end 119.5 80) (width 0.7) (layer "F.Cu") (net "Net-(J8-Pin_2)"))
 (segment (start 143.5 104) (end 143.5 111.04) (width 0.7) (layer "F.Cu") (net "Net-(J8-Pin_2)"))
 (segment (start 143.5 111.04) (end 147 114.54) (width 0.7) (layer "F.Cu") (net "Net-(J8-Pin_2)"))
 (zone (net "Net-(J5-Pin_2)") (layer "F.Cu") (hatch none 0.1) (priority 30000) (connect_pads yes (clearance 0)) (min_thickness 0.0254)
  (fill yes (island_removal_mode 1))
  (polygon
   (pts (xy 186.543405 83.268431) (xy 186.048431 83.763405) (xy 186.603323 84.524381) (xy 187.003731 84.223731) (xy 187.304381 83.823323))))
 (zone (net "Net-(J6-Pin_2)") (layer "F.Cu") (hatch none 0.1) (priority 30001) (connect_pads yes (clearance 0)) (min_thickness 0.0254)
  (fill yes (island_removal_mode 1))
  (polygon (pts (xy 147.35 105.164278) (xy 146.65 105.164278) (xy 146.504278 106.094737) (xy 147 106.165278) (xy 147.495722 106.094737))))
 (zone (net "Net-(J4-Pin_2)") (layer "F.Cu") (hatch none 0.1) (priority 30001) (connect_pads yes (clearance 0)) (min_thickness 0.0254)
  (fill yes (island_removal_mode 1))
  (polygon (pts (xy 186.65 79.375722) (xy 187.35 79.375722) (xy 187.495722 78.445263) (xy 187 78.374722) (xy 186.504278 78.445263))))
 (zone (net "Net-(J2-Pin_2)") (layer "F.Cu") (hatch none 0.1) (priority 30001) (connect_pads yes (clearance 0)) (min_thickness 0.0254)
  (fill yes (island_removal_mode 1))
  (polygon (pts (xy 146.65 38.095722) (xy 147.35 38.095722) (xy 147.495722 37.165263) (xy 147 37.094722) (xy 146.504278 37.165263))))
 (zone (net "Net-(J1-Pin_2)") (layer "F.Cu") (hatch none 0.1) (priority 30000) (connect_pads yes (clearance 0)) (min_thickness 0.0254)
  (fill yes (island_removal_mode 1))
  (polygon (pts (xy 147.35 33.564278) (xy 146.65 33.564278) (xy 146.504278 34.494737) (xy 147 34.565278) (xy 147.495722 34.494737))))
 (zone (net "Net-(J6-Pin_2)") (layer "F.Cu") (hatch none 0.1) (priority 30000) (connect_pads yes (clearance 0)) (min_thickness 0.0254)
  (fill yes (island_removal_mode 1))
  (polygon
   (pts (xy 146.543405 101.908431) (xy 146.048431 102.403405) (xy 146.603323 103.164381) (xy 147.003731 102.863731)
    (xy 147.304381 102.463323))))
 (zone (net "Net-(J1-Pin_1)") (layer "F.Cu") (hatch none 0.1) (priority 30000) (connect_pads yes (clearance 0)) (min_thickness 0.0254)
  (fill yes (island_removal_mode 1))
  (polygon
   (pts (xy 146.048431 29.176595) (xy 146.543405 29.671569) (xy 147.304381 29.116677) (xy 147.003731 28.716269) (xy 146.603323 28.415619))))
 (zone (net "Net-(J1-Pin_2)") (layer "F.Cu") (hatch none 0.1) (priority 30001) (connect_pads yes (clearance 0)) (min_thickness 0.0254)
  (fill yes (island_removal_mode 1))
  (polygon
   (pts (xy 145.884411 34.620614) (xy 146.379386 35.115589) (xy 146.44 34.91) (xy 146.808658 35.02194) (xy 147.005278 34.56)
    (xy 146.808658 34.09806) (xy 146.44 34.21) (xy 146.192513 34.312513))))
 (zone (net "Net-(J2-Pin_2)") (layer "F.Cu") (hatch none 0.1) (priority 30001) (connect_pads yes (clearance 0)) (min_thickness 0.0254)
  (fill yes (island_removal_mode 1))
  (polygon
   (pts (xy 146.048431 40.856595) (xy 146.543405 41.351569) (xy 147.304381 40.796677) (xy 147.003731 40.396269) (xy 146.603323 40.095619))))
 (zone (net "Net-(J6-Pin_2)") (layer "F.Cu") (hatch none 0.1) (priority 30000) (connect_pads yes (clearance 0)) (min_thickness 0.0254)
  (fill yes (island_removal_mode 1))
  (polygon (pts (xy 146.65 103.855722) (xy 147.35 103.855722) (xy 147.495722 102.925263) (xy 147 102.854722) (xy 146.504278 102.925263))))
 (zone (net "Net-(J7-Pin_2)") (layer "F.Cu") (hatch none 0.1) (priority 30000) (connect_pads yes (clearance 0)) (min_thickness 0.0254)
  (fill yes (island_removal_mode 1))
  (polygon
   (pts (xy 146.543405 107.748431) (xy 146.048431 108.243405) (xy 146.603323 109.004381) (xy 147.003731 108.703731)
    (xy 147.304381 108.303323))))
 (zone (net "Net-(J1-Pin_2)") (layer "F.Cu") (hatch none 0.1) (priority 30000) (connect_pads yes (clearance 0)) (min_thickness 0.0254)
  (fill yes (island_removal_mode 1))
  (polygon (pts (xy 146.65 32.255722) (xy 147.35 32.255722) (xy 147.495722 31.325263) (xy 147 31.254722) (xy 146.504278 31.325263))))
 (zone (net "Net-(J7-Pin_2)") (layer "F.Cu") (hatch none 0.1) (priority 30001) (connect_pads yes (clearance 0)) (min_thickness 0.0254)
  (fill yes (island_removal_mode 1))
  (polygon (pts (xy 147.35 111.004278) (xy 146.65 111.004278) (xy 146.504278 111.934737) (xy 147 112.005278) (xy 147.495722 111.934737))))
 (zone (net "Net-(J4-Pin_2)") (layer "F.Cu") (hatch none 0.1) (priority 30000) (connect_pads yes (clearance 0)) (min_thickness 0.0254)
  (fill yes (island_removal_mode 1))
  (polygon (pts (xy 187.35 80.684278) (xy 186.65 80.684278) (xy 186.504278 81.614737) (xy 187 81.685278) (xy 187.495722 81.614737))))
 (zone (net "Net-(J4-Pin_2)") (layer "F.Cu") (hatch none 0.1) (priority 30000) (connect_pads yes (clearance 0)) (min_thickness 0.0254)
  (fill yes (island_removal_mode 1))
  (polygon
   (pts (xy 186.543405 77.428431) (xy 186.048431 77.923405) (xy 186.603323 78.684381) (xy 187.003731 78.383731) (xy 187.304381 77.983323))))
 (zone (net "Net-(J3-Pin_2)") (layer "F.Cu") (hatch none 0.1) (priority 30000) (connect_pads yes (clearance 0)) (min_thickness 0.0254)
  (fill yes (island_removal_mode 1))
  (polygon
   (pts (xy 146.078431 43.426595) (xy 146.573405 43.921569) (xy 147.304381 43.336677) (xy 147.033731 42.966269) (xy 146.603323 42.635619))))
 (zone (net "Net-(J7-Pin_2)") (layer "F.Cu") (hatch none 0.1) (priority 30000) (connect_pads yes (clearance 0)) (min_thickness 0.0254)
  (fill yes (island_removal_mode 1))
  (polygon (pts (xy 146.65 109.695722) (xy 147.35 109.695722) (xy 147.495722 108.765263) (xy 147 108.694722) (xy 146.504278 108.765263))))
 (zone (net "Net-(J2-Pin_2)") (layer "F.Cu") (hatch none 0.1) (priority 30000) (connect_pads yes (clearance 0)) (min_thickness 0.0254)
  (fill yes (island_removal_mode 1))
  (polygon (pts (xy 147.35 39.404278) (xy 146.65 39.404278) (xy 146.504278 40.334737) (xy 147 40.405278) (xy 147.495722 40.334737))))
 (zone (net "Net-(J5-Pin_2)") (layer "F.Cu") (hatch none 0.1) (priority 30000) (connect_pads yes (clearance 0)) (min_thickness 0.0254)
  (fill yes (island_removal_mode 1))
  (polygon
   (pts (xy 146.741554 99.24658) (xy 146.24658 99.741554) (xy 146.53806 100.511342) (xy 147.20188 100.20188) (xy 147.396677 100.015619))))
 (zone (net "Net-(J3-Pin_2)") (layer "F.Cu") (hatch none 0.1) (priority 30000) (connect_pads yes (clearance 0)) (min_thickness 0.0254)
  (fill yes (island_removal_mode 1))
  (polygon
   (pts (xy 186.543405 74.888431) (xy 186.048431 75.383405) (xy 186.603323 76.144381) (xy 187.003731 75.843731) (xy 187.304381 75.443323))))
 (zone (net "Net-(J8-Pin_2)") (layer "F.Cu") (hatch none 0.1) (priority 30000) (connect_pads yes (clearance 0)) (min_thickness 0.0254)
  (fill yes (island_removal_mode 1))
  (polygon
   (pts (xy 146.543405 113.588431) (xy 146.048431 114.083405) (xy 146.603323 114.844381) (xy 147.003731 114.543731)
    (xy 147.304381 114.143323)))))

